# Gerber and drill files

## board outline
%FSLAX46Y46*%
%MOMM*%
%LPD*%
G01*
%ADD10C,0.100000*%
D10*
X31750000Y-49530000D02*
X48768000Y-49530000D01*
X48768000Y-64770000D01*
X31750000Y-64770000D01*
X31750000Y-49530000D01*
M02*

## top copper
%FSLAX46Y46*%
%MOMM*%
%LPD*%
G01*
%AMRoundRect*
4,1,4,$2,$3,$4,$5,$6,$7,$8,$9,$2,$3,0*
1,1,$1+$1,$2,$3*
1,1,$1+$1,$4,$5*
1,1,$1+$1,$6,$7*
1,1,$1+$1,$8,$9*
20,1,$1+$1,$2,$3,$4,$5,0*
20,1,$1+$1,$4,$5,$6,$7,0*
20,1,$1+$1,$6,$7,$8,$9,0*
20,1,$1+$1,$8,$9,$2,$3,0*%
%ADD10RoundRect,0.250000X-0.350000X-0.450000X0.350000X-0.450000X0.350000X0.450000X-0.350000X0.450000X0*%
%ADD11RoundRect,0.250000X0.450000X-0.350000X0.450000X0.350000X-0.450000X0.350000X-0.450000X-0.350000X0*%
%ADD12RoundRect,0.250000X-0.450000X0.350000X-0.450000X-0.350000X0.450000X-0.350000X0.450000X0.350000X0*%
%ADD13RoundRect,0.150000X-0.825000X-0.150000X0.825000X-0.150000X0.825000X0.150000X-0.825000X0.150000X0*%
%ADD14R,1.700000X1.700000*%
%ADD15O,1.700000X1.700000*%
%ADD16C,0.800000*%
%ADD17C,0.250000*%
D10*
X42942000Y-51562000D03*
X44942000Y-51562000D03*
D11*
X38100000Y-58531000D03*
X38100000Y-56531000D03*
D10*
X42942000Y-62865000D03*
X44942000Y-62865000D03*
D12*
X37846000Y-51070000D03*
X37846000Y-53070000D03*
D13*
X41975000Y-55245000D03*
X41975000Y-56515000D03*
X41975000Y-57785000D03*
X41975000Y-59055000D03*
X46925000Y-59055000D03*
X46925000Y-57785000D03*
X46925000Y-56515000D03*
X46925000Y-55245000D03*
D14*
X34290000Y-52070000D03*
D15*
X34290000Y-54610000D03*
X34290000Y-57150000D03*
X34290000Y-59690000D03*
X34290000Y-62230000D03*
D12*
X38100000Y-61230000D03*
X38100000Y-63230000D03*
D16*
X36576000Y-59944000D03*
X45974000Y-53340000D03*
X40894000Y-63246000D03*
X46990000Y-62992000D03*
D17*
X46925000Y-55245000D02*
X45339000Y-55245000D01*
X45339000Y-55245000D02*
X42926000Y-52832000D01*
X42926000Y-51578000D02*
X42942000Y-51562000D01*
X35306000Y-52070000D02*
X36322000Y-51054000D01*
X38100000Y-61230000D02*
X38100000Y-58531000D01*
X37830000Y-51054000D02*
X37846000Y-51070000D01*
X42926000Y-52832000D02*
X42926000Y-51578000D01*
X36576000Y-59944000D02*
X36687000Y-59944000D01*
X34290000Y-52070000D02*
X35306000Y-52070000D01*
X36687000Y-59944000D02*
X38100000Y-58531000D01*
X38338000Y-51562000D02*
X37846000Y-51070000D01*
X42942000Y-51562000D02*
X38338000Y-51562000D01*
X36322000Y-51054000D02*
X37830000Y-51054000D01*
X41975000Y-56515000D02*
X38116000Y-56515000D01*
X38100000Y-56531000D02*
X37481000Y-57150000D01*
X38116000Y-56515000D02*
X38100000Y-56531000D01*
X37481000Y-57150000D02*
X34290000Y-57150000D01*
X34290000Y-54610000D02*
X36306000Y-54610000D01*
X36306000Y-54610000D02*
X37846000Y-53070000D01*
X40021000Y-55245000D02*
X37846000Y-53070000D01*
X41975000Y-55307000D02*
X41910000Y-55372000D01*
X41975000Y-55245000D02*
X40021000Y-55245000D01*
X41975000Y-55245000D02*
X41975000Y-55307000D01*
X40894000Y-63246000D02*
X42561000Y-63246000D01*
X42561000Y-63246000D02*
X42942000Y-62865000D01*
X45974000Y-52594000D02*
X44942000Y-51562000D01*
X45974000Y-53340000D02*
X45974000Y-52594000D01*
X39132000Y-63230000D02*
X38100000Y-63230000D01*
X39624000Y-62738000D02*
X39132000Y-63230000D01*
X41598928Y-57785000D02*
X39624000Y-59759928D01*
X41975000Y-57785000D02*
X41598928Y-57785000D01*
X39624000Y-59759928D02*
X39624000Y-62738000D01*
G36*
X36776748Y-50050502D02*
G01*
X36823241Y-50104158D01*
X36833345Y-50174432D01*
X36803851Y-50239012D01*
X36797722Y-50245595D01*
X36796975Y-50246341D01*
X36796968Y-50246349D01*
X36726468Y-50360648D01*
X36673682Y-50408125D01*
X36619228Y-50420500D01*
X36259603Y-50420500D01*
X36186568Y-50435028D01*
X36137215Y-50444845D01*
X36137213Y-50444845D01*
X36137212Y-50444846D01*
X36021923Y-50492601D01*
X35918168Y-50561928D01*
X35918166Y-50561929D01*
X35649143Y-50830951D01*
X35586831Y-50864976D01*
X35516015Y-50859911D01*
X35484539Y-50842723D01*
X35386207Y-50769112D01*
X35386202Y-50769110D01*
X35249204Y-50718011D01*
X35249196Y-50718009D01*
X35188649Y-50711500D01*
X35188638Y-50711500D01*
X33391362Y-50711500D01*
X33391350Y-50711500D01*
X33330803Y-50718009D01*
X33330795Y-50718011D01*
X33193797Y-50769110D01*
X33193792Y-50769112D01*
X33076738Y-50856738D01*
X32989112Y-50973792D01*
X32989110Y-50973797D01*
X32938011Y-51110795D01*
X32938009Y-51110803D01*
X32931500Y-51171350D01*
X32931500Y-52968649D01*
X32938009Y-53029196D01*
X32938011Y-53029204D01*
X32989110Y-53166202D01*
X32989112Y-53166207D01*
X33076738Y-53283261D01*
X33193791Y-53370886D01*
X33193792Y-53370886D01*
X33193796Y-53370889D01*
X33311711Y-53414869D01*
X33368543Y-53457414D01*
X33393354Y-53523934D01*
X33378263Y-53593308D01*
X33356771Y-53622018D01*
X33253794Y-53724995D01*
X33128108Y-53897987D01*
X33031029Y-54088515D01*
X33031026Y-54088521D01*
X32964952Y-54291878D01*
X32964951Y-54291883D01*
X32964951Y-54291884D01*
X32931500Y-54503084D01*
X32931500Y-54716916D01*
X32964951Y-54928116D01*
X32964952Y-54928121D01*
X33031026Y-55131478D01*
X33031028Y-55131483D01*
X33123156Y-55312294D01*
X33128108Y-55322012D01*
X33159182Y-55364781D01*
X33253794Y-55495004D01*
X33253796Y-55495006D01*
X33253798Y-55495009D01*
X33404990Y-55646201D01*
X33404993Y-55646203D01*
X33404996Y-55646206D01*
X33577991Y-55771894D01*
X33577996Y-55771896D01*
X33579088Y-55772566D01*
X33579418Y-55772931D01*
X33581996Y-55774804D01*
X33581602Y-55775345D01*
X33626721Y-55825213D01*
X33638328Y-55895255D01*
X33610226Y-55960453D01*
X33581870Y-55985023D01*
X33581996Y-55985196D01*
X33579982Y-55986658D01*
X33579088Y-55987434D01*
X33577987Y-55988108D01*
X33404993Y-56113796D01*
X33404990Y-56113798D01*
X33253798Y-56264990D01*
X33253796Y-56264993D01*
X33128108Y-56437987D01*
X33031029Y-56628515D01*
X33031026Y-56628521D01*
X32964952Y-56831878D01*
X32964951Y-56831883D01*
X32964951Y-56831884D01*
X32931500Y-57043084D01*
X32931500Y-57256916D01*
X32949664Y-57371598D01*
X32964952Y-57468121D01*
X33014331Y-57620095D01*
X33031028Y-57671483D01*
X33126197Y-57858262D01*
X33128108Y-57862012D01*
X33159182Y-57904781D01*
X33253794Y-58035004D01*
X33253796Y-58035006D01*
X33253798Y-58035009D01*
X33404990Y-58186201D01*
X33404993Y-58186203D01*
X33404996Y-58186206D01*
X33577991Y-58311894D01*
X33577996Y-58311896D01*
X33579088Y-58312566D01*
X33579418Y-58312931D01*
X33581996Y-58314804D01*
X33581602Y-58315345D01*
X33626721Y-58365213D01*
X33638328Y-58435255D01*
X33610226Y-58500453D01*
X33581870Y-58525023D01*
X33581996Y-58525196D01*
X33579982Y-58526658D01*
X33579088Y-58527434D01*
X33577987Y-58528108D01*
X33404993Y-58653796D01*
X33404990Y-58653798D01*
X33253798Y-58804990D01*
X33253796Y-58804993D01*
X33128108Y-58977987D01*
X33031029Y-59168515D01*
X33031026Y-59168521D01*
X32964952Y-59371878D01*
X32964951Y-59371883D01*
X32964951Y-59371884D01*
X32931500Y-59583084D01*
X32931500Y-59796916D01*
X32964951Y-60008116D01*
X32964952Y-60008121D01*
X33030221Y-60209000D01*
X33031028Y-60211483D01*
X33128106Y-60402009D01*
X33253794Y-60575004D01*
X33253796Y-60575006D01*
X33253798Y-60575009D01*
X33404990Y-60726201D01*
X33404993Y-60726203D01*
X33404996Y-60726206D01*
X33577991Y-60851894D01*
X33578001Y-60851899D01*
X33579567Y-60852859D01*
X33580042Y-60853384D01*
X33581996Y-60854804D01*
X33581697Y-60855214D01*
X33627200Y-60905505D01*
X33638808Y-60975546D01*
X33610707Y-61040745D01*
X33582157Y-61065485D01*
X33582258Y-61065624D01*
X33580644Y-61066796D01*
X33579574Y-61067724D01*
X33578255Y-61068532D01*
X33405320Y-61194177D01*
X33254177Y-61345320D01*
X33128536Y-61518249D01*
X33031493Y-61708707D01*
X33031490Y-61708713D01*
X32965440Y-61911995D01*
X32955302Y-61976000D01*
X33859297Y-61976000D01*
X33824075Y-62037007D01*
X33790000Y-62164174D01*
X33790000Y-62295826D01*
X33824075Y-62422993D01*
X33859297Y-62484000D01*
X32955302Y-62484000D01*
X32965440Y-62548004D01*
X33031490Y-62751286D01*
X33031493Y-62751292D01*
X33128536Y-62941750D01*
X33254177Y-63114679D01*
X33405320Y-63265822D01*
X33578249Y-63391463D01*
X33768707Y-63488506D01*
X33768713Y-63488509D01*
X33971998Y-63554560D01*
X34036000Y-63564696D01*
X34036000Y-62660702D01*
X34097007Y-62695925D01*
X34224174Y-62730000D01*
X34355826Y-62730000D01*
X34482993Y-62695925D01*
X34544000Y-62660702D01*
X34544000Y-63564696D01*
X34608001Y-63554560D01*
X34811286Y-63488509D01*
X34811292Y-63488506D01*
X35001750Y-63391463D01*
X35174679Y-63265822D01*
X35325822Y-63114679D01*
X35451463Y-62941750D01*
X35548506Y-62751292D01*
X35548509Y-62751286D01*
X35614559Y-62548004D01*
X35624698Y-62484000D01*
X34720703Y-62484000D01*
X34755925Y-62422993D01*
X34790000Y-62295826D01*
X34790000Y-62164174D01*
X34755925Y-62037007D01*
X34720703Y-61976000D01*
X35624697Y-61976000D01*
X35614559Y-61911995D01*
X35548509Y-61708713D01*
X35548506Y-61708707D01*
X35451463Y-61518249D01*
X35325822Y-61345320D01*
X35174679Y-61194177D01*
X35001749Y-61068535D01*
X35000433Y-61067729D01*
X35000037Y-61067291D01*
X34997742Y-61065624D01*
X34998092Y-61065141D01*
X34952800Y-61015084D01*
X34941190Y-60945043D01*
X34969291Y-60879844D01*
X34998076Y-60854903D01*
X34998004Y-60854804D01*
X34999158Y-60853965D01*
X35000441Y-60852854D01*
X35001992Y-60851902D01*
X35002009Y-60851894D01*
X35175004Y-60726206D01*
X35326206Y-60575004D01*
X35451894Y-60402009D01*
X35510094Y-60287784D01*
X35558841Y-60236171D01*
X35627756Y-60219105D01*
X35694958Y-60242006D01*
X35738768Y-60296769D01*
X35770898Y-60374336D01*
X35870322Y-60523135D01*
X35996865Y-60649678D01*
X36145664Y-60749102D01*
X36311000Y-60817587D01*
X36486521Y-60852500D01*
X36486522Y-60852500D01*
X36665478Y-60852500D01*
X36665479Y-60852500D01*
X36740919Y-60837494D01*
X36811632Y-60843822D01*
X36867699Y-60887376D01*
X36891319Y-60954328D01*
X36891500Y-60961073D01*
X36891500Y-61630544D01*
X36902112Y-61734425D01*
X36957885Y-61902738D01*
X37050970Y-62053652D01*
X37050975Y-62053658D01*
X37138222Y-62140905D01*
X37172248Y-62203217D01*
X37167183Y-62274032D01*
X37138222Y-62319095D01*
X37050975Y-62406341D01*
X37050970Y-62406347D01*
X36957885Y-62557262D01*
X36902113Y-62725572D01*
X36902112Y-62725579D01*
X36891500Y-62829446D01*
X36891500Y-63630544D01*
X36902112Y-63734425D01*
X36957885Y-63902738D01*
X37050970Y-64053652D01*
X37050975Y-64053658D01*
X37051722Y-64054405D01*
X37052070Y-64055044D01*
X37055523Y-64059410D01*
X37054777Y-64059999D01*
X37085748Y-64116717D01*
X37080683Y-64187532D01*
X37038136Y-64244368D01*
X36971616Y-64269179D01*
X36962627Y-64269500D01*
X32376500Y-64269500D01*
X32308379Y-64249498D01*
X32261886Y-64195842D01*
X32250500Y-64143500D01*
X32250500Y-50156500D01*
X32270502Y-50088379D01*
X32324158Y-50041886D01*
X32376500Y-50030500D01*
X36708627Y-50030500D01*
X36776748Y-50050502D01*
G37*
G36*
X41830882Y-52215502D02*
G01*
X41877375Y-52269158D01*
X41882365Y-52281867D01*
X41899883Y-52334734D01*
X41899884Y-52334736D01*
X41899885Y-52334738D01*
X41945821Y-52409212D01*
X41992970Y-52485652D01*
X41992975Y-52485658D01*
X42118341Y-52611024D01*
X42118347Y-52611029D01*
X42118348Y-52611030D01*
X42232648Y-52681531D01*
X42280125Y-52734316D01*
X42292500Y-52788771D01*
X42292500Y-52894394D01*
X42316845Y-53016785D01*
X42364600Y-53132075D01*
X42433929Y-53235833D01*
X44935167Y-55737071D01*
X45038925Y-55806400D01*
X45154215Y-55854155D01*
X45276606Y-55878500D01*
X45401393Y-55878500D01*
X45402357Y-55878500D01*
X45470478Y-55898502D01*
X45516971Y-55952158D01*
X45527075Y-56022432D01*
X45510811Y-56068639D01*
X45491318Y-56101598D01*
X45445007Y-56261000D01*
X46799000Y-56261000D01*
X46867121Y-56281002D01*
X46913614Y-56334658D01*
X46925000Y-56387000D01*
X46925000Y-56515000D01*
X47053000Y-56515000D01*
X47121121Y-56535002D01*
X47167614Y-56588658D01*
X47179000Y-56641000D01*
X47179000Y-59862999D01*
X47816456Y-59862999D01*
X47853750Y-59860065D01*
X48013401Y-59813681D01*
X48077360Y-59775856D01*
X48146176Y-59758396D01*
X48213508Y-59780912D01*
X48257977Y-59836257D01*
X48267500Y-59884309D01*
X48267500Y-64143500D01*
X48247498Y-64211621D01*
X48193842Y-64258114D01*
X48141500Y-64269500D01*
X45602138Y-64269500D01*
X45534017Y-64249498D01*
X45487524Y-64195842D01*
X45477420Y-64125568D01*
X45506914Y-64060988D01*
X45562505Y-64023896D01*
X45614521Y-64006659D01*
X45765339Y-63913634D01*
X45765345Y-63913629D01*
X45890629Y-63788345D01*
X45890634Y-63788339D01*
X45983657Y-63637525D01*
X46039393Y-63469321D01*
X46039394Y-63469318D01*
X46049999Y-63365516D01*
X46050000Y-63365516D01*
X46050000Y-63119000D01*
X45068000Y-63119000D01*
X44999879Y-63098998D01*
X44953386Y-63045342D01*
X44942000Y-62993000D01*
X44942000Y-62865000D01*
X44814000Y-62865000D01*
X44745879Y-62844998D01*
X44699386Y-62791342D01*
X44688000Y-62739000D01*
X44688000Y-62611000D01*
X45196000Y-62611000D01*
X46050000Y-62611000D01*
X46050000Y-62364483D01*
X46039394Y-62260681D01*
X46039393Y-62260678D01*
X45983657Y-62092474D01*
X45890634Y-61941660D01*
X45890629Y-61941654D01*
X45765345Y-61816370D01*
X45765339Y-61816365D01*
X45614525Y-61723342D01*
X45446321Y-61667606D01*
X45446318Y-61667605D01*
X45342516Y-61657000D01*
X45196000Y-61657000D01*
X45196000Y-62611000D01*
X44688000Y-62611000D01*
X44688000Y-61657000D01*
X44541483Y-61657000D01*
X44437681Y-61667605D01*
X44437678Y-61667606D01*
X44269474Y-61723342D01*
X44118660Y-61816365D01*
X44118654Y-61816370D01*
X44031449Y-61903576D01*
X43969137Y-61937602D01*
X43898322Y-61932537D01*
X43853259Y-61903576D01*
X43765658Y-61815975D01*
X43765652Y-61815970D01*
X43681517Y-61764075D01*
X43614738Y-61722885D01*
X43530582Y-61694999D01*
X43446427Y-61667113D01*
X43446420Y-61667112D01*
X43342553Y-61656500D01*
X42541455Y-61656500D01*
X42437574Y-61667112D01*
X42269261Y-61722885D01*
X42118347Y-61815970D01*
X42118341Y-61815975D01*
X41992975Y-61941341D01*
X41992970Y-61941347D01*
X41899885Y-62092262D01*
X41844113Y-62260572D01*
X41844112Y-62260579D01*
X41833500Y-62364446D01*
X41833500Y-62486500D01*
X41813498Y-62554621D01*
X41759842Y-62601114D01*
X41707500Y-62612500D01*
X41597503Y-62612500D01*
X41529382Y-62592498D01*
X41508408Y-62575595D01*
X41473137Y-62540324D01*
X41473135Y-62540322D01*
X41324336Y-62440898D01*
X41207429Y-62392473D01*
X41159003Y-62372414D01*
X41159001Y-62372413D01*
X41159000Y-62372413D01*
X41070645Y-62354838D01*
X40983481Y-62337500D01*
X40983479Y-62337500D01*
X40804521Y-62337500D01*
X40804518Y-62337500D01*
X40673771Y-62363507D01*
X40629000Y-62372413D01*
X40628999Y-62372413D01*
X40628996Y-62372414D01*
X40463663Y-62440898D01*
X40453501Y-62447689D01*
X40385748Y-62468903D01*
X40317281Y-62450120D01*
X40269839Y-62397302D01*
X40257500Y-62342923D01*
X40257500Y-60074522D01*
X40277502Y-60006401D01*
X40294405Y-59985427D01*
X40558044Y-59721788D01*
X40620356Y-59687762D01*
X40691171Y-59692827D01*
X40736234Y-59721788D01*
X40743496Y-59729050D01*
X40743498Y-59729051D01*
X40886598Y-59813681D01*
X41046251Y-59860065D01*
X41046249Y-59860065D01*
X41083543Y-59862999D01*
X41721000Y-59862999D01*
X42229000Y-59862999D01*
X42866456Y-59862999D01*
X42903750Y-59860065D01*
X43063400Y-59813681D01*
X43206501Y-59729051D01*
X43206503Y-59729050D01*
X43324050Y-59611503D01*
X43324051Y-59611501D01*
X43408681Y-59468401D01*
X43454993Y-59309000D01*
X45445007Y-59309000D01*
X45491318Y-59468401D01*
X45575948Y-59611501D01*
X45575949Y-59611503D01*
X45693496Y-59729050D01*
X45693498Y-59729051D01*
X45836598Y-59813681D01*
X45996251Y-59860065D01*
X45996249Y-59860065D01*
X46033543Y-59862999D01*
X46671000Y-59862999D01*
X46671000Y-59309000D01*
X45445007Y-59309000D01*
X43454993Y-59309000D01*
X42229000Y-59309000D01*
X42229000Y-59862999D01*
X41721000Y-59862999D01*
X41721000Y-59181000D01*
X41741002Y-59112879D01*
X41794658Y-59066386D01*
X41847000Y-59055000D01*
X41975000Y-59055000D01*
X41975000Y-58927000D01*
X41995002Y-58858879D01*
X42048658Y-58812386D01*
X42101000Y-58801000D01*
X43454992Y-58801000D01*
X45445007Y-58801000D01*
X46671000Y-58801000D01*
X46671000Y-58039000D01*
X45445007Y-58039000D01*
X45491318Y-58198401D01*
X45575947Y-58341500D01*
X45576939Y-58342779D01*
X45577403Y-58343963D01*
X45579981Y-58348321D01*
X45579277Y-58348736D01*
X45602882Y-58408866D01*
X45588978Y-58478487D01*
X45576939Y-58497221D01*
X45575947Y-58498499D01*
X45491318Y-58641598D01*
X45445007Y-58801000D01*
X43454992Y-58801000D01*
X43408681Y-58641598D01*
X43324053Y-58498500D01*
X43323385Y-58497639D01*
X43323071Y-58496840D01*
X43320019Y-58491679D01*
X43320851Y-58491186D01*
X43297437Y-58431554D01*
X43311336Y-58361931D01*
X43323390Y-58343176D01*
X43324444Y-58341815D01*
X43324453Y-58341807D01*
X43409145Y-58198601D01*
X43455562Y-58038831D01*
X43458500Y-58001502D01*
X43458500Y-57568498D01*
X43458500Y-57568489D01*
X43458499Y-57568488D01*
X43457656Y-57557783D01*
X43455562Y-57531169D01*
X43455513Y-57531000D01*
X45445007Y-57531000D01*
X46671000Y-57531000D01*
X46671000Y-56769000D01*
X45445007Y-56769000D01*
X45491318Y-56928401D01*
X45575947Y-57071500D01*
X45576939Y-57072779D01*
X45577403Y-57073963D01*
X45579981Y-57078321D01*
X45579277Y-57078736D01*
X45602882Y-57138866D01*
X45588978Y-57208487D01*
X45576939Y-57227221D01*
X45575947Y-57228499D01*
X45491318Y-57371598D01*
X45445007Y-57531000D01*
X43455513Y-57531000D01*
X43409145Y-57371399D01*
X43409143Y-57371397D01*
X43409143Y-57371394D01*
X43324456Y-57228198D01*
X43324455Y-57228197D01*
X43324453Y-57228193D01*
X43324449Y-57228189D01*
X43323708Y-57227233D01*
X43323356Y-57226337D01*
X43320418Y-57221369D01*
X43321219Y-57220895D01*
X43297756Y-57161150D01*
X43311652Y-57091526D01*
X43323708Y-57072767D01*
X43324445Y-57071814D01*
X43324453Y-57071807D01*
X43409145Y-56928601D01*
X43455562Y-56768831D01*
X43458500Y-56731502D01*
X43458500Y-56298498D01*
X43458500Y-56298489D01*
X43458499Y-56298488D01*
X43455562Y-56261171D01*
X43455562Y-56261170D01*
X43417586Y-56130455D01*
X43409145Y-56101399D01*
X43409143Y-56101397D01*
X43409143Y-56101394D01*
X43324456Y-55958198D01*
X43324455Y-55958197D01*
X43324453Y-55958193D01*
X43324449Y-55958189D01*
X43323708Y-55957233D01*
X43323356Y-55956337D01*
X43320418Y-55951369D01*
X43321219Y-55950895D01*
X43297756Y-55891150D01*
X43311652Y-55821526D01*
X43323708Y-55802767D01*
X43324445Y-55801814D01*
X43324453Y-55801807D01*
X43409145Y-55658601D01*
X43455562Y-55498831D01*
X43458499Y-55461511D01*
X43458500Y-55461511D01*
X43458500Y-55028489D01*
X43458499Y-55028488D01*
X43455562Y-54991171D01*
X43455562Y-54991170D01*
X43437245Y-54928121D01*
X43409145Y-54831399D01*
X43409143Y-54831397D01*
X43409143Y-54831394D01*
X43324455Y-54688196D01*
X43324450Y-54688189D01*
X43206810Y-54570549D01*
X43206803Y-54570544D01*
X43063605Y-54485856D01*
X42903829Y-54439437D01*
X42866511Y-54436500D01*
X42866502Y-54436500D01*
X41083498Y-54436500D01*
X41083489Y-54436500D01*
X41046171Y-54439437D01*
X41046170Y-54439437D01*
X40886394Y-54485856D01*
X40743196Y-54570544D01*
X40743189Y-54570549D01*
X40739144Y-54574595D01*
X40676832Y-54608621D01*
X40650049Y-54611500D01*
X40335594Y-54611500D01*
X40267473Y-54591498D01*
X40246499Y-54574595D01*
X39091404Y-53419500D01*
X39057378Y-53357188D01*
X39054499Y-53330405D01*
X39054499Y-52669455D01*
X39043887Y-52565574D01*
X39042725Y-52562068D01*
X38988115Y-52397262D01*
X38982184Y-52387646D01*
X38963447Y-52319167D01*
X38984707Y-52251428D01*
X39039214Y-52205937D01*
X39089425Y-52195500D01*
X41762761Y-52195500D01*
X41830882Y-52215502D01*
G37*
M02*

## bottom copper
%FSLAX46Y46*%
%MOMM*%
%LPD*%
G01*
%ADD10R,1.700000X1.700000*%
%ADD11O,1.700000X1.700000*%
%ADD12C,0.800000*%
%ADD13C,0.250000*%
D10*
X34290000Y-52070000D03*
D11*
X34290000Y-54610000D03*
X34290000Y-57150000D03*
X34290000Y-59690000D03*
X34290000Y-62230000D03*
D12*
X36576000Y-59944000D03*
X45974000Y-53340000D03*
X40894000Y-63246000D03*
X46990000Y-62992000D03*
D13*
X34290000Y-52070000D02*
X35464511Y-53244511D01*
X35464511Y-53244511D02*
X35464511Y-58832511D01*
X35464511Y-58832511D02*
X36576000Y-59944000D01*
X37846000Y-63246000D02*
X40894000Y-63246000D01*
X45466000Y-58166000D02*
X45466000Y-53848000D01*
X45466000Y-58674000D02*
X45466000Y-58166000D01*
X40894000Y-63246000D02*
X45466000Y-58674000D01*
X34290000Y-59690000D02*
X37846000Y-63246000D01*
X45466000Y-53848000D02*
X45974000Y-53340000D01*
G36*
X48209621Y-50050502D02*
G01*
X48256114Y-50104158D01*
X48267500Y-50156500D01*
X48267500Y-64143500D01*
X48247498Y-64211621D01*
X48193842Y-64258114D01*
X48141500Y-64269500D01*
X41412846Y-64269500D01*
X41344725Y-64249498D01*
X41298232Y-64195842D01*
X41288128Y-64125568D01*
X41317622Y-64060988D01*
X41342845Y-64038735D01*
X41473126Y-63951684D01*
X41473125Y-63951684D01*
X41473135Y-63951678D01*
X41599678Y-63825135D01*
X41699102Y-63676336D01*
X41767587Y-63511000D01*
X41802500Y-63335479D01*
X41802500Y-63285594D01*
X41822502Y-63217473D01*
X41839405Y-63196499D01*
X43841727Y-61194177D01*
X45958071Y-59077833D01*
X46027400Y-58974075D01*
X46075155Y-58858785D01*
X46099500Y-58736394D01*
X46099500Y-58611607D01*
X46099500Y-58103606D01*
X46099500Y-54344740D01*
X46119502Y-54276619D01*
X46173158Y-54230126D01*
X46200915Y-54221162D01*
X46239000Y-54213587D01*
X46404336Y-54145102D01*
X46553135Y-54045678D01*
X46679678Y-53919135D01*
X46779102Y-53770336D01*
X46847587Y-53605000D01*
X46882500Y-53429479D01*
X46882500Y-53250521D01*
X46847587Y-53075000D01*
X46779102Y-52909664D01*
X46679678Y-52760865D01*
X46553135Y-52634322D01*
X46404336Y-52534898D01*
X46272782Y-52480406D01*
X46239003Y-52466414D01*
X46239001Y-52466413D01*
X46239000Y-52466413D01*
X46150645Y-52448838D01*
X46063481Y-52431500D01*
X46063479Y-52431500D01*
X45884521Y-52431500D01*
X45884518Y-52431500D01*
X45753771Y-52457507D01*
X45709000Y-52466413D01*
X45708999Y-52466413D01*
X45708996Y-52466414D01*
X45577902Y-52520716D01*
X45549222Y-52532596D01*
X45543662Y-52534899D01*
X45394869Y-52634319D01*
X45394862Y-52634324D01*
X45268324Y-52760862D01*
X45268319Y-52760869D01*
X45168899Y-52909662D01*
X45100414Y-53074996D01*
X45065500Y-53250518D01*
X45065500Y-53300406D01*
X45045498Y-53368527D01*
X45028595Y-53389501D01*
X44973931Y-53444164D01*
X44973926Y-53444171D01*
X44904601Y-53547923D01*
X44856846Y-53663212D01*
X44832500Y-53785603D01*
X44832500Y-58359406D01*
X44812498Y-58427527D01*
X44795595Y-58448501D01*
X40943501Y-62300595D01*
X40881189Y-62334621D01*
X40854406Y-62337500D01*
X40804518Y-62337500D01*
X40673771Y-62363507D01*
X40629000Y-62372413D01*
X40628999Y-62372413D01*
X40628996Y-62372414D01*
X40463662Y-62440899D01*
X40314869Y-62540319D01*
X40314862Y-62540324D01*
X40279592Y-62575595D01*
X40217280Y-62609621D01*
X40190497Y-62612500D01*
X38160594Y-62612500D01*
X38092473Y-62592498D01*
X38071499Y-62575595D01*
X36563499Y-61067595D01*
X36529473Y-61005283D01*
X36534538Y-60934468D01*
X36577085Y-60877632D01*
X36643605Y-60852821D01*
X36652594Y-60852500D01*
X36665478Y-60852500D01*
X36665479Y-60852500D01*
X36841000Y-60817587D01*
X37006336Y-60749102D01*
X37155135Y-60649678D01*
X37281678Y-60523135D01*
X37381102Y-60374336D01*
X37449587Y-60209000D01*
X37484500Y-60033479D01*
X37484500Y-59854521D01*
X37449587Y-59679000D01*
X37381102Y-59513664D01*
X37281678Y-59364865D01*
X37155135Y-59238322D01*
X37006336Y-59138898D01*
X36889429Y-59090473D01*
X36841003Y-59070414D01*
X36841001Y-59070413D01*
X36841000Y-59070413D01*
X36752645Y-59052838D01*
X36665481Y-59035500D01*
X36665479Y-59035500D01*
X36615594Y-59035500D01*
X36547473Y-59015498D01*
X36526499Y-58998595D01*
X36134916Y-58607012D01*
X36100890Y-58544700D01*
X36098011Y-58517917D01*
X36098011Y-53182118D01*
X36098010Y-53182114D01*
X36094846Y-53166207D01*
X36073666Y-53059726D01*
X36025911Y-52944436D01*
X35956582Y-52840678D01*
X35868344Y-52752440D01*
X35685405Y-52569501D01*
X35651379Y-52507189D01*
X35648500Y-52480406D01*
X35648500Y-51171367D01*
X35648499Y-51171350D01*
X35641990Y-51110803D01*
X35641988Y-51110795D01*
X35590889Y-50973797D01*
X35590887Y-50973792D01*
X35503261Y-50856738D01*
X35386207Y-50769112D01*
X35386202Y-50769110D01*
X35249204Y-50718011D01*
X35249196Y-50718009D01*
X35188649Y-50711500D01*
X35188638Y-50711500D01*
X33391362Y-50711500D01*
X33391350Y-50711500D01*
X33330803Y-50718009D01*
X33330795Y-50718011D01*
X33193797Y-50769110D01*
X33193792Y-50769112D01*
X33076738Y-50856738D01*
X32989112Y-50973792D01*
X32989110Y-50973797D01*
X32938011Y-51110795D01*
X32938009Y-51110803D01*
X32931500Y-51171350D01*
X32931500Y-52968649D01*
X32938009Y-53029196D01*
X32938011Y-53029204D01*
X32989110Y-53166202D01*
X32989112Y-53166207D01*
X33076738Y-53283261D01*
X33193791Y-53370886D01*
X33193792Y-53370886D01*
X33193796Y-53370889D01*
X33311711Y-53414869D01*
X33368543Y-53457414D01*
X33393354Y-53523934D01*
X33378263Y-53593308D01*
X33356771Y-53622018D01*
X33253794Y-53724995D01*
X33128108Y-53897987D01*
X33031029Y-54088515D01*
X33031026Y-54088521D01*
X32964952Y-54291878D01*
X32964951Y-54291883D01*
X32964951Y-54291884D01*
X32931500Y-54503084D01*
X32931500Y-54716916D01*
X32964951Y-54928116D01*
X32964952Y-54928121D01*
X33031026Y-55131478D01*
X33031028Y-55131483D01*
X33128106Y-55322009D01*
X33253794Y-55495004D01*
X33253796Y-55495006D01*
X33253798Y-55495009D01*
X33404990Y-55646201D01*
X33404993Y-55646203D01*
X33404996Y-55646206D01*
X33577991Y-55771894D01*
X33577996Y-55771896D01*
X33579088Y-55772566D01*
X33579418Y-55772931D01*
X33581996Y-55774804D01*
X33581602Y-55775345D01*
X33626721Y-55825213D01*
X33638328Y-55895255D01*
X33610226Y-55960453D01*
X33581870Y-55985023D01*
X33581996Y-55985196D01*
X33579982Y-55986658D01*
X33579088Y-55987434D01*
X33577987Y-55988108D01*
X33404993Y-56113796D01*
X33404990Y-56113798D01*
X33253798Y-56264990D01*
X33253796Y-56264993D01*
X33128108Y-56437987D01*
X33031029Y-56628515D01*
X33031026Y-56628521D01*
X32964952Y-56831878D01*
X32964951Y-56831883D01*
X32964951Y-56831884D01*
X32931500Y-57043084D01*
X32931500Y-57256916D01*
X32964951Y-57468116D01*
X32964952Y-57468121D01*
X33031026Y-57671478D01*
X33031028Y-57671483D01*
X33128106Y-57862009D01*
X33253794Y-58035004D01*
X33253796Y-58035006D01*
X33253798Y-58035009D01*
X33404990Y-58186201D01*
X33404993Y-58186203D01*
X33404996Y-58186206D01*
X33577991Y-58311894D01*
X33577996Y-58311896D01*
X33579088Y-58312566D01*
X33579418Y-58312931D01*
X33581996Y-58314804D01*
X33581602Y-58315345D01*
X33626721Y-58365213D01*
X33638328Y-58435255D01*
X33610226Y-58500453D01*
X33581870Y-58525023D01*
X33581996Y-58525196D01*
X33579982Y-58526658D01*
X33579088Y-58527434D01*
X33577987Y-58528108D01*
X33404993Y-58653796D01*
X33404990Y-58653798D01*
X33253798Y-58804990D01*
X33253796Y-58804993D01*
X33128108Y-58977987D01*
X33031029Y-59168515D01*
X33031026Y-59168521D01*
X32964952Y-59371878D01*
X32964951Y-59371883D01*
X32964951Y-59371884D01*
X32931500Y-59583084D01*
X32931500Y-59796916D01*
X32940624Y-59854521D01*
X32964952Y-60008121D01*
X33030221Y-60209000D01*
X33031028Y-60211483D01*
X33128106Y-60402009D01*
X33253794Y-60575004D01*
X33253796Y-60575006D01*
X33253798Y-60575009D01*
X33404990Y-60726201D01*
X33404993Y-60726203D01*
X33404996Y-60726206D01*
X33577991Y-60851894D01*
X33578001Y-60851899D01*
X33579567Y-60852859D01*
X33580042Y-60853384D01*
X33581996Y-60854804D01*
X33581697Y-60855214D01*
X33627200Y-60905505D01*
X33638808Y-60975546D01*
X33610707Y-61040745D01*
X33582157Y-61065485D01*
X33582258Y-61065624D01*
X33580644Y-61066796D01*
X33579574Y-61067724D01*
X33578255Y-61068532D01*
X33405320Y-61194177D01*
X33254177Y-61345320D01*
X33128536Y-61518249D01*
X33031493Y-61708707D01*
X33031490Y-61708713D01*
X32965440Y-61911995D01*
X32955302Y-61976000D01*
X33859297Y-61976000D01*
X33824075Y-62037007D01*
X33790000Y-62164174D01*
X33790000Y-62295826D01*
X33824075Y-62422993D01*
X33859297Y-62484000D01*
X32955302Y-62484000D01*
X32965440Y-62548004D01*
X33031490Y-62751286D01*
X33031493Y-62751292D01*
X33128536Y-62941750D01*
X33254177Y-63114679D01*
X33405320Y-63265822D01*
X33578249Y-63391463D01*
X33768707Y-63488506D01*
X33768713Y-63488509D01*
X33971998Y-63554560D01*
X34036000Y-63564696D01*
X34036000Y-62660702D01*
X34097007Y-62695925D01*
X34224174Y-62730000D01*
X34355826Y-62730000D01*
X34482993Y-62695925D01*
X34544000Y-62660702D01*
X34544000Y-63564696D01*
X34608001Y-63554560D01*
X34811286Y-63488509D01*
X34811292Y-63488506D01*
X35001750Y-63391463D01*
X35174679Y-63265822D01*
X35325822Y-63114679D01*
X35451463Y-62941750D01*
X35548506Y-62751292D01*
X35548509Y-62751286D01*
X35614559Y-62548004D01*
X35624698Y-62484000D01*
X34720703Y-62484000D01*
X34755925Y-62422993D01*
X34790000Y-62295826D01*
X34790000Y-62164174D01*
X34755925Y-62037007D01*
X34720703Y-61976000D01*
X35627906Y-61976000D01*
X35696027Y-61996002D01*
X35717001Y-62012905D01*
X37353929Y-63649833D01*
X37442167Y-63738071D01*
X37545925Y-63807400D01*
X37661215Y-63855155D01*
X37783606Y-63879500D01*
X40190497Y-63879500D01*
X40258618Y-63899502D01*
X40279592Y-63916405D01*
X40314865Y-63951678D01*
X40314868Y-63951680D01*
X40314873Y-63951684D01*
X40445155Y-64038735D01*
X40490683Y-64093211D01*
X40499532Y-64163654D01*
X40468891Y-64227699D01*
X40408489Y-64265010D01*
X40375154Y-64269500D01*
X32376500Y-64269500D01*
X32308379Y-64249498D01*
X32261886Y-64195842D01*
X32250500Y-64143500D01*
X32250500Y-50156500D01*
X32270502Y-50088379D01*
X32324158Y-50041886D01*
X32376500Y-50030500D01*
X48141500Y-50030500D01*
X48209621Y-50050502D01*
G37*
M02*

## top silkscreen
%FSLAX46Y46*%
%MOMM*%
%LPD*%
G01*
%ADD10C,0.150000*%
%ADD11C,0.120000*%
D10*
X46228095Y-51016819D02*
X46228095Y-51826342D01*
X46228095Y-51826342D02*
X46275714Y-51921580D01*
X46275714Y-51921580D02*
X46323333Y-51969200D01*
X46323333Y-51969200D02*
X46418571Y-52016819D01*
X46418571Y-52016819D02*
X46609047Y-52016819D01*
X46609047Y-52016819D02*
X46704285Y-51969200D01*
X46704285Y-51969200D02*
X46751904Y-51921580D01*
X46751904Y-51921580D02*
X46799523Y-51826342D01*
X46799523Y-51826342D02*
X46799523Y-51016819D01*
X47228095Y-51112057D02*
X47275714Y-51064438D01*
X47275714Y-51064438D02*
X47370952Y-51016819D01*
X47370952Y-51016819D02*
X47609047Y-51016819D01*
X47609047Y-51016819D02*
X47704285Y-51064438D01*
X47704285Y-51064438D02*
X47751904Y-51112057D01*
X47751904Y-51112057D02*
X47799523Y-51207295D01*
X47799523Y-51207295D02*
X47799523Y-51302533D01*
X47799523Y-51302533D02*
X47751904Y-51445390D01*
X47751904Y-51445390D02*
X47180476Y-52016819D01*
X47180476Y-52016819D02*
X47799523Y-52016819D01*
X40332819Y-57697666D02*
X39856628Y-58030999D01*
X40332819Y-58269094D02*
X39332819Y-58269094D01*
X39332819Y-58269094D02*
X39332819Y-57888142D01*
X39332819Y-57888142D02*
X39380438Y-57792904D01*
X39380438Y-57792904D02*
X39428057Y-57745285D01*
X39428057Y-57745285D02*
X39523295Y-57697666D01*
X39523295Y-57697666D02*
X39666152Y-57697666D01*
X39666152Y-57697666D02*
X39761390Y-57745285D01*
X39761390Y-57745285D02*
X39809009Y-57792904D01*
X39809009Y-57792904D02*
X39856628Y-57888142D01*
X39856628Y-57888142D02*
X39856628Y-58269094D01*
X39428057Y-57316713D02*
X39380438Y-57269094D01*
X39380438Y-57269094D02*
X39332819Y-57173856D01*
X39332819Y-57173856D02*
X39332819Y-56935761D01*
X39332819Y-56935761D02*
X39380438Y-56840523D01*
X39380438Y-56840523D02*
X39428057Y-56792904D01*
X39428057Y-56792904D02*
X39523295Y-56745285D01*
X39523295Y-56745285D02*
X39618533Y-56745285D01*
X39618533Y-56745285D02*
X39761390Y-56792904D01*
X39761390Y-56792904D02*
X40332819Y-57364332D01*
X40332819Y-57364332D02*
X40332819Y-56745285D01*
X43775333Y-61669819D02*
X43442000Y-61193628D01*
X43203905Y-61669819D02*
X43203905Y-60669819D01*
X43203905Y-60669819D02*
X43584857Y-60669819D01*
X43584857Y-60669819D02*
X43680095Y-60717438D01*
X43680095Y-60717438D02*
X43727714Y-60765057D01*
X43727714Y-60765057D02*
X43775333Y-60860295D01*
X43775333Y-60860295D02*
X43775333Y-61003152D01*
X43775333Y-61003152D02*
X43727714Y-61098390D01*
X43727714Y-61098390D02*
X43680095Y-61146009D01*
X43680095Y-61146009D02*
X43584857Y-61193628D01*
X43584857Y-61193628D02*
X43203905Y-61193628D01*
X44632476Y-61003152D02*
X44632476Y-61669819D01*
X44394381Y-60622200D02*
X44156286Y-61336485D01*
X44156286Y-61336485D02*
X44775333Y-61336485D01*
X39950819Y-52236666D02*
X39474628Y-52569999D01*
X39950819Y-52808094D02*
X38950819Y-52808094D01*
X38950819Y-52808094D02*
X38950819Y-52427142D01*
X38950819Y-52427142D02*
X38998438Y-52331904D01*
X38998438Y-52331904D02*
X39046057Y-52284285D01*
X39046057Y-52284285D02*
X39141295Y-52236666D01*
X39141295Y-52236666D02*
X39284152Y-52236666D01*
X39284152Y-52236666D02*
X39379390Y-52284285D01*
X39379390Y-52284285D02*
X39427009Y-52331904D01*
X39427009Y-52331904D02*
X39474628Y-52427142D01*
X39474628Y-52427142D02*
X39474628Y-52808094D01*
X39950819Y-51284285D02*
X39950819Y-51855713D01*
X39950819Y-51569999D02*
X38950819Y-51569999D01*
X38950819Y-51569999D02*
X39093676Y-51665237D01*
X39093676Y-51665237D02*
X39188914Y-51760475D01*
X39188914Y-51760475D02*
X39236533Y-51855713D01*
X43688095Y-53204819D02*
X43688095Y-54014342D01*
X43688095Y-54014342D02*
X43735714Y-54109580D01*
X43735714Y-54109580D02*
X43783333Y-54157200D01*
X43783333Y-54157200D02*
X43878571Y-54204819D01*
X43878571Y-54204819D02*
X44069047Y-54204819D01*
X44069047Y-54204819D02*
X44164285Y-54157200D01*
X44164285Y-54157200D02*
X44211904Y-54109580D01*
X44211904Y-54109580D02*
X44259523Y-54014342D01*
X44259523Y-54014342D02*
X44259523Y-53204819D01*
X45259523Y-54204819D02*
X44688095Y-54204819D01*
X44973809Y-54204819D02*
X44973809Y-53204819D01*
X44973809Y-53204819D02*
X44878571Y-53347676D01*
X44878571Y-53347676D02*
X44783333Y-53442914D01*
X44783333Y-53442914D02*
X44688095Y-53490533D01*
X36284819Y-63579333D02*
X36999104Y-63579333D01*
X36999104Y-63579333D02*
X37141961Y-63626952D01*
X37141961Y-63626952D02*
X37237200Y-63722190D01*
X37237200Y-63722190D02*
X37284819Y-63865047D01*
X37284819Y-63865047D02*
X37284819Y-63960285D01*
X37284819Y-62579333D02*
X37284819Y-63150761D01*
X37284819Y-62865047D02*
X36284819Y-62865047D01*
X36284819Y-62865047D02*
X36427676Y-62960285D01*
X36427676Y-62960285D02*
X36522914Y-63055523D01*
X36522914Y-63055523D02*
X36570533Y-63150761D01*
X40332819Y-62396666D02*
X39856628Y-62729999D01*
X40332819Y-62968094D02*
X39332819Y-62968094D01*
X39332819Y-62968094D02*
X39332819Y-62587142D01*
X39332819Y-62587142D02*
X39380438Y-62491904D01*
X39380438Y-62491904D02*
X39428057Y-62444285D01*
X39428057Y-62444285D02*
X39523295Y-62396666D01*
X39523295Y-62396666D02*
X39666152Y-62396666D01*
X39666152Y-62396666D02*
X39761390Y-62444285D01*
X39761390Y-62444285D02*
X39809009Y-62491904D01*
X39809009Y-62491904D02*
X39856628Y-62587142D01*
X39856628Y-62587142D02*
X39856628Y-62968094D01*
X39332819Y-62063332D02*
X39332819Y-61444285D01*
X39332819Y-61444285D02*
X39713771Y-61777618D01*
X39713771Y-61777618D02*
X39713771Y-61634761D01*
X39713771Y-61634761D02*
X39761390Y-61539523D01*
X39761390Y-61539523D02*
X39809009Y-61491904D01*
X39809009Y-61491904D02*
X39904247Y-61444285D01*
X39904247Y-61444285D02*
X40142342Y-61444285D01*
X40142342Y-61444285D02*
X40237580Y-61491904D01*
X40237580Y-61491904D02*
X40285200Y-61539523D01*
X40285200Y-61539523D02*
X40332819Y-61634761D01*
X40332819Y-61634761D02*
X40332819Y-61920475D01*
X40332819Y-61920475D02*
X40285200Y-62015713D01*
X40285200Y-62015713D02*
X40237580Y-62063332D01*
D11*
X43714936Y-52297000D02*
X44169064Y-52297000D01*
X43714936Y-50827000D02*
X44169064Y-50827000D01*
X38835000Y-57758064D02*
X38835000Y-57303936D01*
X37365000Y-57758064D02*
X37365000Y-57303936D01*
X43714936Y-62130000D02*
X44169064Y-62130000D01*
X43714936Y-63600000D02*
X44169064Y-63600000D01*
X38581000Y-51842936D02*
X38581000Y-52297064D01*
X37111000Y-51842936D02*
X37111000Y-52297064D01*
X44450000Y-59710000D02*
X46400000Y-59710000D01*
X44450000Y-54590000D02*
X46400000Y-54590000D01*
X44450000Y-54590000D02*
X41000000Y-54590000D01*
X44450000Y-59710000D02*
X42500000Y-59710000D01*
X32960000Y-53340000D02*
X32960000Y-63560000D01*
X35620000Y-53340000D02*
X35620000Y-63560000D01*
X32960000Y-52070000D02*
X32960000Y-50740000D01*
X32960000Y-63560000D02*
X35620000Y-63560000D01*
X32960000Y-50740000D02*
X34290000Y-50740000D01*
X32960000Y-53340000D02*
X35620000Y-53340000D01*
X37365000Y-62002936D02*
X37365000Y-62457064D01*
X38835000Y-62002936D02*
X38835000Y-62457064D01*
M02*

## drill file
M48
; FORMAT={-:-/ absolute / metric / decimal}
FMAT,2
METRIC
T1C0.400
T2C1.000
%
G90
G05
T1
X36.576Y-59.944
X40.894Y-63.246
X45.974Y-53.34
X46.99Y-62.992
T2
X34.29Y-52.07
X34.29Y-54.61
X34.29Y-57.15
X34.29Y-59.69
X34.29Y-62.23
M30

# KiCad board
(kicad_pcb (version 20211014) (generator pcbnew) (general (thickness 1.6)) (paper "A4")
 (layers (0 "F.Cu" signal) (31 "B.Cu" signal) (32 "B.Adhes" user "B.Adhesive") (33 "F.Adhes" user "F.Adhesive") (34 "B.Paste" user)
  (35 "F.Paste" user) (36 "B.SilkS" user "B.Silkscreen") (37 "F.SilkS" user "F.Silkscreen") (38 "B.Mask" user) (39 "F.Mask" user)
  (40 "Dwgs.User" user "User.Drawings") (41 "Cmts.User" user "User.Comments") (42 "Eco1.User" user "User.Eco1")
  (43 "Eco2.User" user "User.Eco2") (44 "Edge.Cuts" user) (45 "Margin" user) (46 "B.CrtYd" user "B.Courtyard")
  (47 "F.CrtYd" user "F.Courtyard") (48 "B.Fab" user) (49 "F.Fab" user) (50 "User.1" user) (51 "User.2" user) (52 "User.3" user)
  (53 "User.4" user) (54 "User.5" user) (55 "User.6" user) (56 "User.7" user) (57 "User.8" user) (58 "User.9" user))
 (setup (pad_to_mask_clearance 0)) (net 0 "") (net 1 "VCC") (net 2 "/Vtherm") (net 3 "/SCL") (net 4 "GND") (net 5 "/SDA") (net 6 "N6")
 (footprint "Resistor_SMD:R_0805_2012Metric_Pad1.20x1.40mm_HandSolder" (layer "F.Cu") (at 43.942 51.562)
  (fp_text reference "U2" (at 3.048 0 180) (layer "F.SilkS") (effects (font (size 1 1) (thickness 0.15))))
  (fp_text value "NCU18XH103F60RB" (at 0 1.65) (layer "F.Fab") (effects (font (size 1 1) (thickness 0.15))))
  (fp_line (start -0.227064 0.735) (end 0.227064 0.735) (layer "F.SilkS") (width 0.12))
  (fp_line (start -0.227064 -0.735) (end 0.227064 -0.735) (layer "F.SilkS") (width 0.12))
  (pad "1" smd roundrect (at -1 0) (size 1.2 1.4) (layers "F.Cu" "F.Paste" "F.Mask") (roundrect_rratio 0.2083333333) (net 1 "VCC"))
  (pad "2" smd roundrect (at 1 0) (size 1.2 1.4) (layers "F.Cu" "F.Paste" "F.Mask") (roundrect_rratio 0.2083333333) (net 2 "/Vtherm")))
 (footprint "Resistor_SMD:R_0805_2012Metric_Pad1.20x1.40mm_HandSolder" (layer "F.Cu") (at 38.1 57.531 90)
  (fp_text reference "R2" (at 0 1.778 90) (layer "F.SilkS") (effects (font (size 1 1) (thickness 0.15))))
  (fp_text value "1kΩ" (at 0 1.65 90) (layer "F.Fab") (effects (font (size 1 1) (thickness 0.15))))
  (fp_line (start -0.227064 0.735) (end 0.227064 0.735) (layer "F.SilkS") (width 0.12))
  (fp_line (start -0.227064 -0.735) (end 0.227064 -0.735) (layer "F.SilkS") (width 0.12))
  (pad "1" smd roundrect (at -1 0 90) (size 1.2 1.4) (layers "F.Cu" "F.Paste" "F.Mask") (roundrect_rratio 0.2083333333) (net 1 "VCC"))
  (pad "2" smd roundrect (at 1 0 90) (size 1.2 1.4) (layers "F.Cu" "F.Paste" "F.Mask") (roundrect_rratio 0.2083333333) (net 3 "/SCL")))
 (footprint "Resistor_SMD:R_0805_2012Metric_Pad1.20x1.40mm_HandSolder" (layer "F.Cu") (at 43.942 62.865)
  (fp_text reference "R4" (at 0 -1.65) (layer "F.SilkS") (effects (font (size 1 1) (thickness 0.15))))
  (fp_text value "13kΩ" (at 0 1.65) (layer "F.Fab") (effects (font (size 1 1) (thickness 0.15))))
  (fp_line (start -0.227064 -0.735) (end 0.227064 -0.735) (layer "F.SilkS") (width 0.12))
  (fp_line (start -0.227064 0.735) (end 0.227064 0.735) (layer "F.SilkS") (width 0.12))
  (pad "1" smd roundrect (at -1 0) (size 1.2 1.4) (layers "F.Cu" "F.Paste" "F.Mask") (roundrect_rratio 0.2083333333) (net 2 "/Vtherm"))
  (pad "2" smd roundrect (at 1 0) (size 1.2 1.4) (layers "F.Cu" "F.Paste" "F.Mask") (roundrect_rratio 0.2083333333) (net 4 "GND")))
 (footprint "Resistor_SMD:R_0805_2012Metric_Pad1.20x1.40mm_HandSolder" (layer "F.Cu") (at 37.846 52.07 -90)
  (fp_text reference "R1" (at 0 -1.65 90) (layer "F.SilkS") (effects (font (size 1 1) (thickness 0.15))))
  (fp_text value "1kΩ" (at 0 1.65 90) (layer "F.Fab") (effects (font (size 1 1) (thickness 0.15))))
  (fp_line (start -0.227064 -0.735) (end 0.227064 -0.735) (layer "F.SilkS") (width 0.12))
  (fp_line (start -0.227064 0.735) (end 0.227064 0.735) (layer "F.SilkS") (width 0.12))
  (pad "1" smd roundrect (at -1 0 270) (size 1.2 1.4) (layers "F.Cu" "F.Paste" "F.Mask") (roundrect_rratio 0.2083333333) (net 1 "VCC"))
  (pad "2" smd roundrect (at 1 0 270) (size 1.2 1.4) (layers "F.Cu" "F.Paste" "F.Mask") (roundrect_rratio 0.2083333333) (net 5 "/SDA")))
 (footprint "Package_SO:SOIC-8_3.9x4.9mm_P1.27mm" (layer "F.Cu") (at 44.45 57.15)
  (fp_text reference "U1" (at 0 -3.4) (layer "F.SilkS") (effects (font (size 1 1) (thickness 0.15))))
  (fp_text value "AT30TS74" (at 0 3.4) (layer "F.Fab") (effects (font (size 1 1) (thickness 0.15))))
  (fp_line (start 0 2.56) (end 1.95 2.56) (layer "F.SilkS") (width 0.12))
  (fp_line (start 0 -2.56) (end 1.95 -2.56) (layer "F.SilkS") (width 0.12))
  (fp_line (start 0 -2.56) (end -3.45 -2.56) (layer "F.SilkS") (width 0.12))
  (fp_line (start 0 2.56) (end -1.95 2.56) (layer "F.SilkS") (width 0.12))
  (pad "1" smd roundrect (at -2.475 -1.905) (size 1.95 0.6) (layers "F.Cu" "F.Paste" "F.Mask") (roundrect_rratio 0.25) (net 5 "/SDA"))
  (pad "2" smd roundrect (at -2.475 -0.635) (size 1.95 0.6) (layers "F.Cu" "F.Paste" "F.Mask") (roundrect_rratio 0.25) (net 3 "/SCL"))
  (pad "3" smd roundrect (at -2.475 0.635) (size 1.95 0.6) (layers "F.Cu" "F.Paste" "F.Mask") (roundrect_rratio 0.25) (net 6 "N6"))
  (pad "4" smd roundrect (at -2.475 1.905) (size 1.95 0.6) (layers "F.Cu" "F.Paste" "F.Mask") (roundrect_rratio 0.25) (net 4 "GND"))
  (pad "5" smd roundrect (at 2.475 1.905) (size 1.95 0.6) (layers "F.Cu" "F.Paste" "F.Mask") (roundrect_rratio 0.25) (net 4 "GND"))
  (pad "6" smd roundrect (at 2.475 0.635) (size 1.95 0.6) (layers "F.Cu" "F.Paste" "F.Mask") (roundrect_rratio 0.25) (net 4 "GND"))
  (pad "7" smd roundrect (at 2.475 -0.635) (size 1.95 0.6) (layers "F.Cu" "F.Paste" "F.Mask") (roundrect_rratio 0.25) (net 4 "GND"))
  (pad "8" smd roundrect (at 2.475 -1.905) (size 1.95 0.6) (layers "F.Cu" "F.Paste" "F.Mask") (roundrect_rratio 0.25) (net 1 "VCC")))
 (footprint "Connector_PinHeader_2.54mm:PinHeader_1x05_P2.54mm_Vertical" (layer "F.Cu") (at 34.29 52.07)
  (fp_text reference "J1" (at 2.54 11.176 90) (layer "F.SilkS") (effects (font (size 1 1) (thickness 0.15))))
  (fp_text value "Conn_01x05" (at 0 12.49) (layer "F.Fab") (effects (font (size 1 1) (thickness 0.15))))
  (fp_line (start -1.33 1.27) (end -1.33 11.49) (layer "F.SilkS") (width 0.12))
  (fp_line (start 1.33 1.27) (end 1.33 11.49) (layer "F.SilkS") (width 0.12))
  (fp_line (start -1.33 0) (end -1.33 -1.33) (layer "F.SilkS") (width 0.12))
  (fp_line (start -1.33 11.49) (end 1.33 11.49) (layer "F.SilkS") (width 0.12))
  (fp_line (start -1.33 -1.33) (end 0 -1.33) (layer "F.SilkS") (width 0.12))
  (fp_line (start -1.33 1.27) (end 1.33 1.27) (layer "F.SilkS") (width 0.12))
  (pad "1" thru_hole rect (at 0 0) (size 1.7 1.7) (drill 1) (layers *.Cu *.Mask) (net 1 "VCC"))
  (pad "2" thru_hole oval (at 0 2.54) (size 1.7 1.7) (drill 1) (layers *.Cu *.Mask) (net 5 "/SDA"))
  (pad "3" thru_hole oval (at 0 5.08) (size 1.7 1.7) (drill 1) (layers *.Cu *.Mask) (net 3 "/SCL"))
  (pad "4" thru_hole oval (at 0 7.62) (size 1.7 1.7) (drill 1) (layers *.Cu *.Mask) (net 2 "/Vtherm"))
  (pad "5" thru_hole oval (at 0 10.16) (size 1.7 1.7) (drill 1) (layers *.Cu *.Mask) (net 4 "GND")))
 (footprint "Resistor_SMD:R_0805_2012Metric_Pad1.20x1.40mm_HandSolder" (layer "F.Cu") (at 38.1 62.23 -90)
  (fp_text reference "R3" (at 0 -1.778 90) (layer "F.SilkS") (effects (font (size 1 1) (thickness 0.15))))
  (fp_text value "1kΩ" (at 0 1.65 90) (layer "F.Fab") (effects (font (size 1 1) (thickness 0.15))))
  (fp_line (start -0.227064 0.735) (end 0.227064 0.735) (layer "F.SilkS") (width 0.12))
  (fp_line (start -0.227064 -0.735) (end 0.227064 -0.735) (layer "F.SilkS") (width 0.12))
  (pad "1" smd roundrect (at -1 0 270) (size 1.2 1.4) (layers "F.Cu" "F.Paste" "F.Mask") (roundrect_rratio 0.2083333333) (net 1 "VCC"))
  (pad "2" smd roundrect (at 1 0 270) (size 1.2 1.4) (layers "F.Cu" "F.Paste" "F.Mask") (roundrect_rratio 0.2083333333) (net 6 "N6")))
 (gr_rect (start 48.768 64.77) (end 31.75 49.53) (layer "Edge.Cuts") (width 0.1) (fill none))
 (segment (start 46.925 55.245) (end 45.339 55.245) (width 0.25) (layer "F.Cu") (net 1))
 (segment (start 45.339 55.245) (end 42.926 52.832) (width 0.25) (layer "F.Cu") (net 1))
 (segment (start 42.926 51.578) (end 42.942 51.562) (width 0.25) (layer "F.Cu") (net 1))
 (segment (start 35.306 52.07) (end 36.322 51.054) (width 0.25) (layer "F.Cu") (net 1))
 (segment (start 38.1 61.23) (end 38.1 58.531) (width 0.25) (layer "F.Cu") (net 1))
 (segment (start 37.83 51.054) (end 37.846 51.07) (width 0.25) (layer "F.Cu") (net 1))
 (segment (start 42.926 52.832) (end 42.926 51.578) (width 0.25) (layer "F.Cu") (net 1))
 (segment (start 36.576 59.944) (end 36.687 59.944) (width 0.25) (layer "F.Cu") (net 1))
 (segment (start 34.29 52.07) (end 35.306 52.07) (width 0.25) (layer "F.Cu") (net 1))
 (segment (start 36.687 59.944) (end 38.1 58.531) (width 0.25) (layer "F.Cu") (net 1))
 (segment (start 38.338 51.562) (end 37.846 51.07) (width 0.25) (layer "F.Cu") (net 1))
 (segment (start 42.942 51.562) (end 38.338 51.562) (width 0.25) (layer "F.Cu") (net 1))
 (segment (start 36.322 51.054) (end 37.83 51.054) (width 0.25) (layer "F.Cu") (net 1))
 (via (at 36.576 59.944) (size 0.8) (drill 0.4) (layers "F.Cu" "B.Cu") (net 1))
 (segment (start 34.29 52.07) (end 35.464511 53.244511) (width 0.25) (layer "B.Cu") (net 1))
 (segment (start 35.464511 53.244511) (end 35.464511 58.832511) (width 0.25) (layer "B.Cu") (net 1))
 (segment (start 35.464511 58.832511) (end 36.576 59.944) (width 0.25) (layer "B.Cu") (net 1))
 (segment (start 41.975 56.515) (end 38.116 56.515) (width 0.25) (layer "F.Cu") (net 3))
 (segment (start 38.1 56.531) (end 37.481 57.15) (width 0.25) (layer "F.Cu") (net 3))
 (segment (start 38.116 56.515) (end 38.1 56.531) (width 0.25) (layer "F.Cu") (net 3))
 (segment (start 37.481 57.15) (end 34.29 57.15) (width 0.25) (layer "F.Cu") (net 3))
 (segment (start 34.29 54.61) (end 36.306 54.61) (width 0.25) (layer "F.Cu") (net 5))
 (segment (start 36.306 54.61) (end 37.846 53.07) (width 0.25) (layer "F.Cu") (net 5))
 (segment (start 40.021 55.245) (end 37.846 53.07) (width 0.25) (layer "F.Cu") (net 5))
 (segment (start 41.975 55.307) (end 41.91 55.372) (width 0.25) (layer "F.Cu") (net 5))
 (segment (start 41.975 55.245) (end 40.021 55.245) (width 0.25) (layer "F.Cu") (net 5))
 (segment (start 41.975 55.245) (end 41.975 55.307) (width 0.25) (layer "F.Cu") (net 5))
 (segment (start 40.894 63.246) (end 42.561 63.246) (width 0.25) (layer "F.Cu") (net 2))
 (segment (start 42.561 63.246) (end 42.942 62.865) (width 0.25) (layer "F.Cu") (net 2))
 (segment (start 45.974 52.594) (end 44.942 51.562) (width 0.25) (layer "F.Cu") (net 2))
 (segment (start 45.974 53.34) (end 45.974 52.594) (width 0.25) (layer "F.Cu") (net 2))
 (via (at 45.974 53.34) (size 0.8) (drill 0.4) (layers "F.Cu" "B.Cu") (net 2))
 (via (at 40.894 63.246) (size 0.8) (drill 0.4) (layers "F.Cu" "B.Cu") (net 2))
 (segment (start 37.846 63.246) (end 40.894 63.246) (width 0.25) (layer "B.Cu") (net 2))
 (segment (start 45.466 58.166) (end 45.466 53.848) (width 0.25) (layer "B.Cu") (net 2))
 (segment (start 45.466 58.674) (end 45.466 58.166) (width 0.25) (layer "B.Cu") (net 2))
 (segment (start 40.894 63.246) (end 45.466 58.674) (width 0.25) (layer "B.Cu") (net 2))
 (segment (start 34.29 59.69) (end 37.846 63.246) (width 0.25) (layer "B.Cu") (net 2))
 (segment (start 45.466 53.848) (end 45.974 53.34) (width 0.25) (layer "B.Cu") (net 2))
 (via (at 46.99 62.992) (size 0.8) (drill 0.4) (layers "F.Cu" "B.Cu") (free) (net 4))
 (segment (start 39.132 63.23) (end 38.1 63.23) (width 0.25) (layer "F.Cu") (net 6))
 (segment (start 39.624 62.738) (end 39.132 63.23) (width 0.25) (layer "F.Cu") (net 6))
 (segment (start 41.598928 57.785) (end 39.624 59.759928) (width 0.25) (layer "F.Cu") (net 6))
 (segment (start 41.975 57.785) (end 41.598928 57.785) (width 0.25) (layer "F.Cu") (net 6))
 (segment (start 39.624 59.759928) (end 39.624 62.738) (width 0.25) (layer "F.Cu") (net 6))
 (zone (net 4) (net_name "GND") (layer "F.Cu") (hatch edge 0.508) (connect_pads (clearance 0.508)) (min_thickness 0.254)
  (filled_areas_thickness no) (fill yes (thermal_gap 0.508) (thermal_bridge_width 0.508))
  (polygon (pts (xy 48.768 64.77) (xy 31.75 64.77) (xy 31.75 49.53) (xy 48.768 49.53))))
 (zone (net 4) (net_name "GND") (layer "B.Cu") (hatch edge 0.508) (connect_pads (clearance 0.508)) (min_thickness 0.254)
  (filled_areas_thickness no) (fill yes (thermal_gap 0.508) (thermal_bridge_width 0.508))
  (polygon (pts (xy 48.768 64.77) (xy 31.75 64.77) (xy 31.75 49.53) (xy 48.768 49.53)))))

